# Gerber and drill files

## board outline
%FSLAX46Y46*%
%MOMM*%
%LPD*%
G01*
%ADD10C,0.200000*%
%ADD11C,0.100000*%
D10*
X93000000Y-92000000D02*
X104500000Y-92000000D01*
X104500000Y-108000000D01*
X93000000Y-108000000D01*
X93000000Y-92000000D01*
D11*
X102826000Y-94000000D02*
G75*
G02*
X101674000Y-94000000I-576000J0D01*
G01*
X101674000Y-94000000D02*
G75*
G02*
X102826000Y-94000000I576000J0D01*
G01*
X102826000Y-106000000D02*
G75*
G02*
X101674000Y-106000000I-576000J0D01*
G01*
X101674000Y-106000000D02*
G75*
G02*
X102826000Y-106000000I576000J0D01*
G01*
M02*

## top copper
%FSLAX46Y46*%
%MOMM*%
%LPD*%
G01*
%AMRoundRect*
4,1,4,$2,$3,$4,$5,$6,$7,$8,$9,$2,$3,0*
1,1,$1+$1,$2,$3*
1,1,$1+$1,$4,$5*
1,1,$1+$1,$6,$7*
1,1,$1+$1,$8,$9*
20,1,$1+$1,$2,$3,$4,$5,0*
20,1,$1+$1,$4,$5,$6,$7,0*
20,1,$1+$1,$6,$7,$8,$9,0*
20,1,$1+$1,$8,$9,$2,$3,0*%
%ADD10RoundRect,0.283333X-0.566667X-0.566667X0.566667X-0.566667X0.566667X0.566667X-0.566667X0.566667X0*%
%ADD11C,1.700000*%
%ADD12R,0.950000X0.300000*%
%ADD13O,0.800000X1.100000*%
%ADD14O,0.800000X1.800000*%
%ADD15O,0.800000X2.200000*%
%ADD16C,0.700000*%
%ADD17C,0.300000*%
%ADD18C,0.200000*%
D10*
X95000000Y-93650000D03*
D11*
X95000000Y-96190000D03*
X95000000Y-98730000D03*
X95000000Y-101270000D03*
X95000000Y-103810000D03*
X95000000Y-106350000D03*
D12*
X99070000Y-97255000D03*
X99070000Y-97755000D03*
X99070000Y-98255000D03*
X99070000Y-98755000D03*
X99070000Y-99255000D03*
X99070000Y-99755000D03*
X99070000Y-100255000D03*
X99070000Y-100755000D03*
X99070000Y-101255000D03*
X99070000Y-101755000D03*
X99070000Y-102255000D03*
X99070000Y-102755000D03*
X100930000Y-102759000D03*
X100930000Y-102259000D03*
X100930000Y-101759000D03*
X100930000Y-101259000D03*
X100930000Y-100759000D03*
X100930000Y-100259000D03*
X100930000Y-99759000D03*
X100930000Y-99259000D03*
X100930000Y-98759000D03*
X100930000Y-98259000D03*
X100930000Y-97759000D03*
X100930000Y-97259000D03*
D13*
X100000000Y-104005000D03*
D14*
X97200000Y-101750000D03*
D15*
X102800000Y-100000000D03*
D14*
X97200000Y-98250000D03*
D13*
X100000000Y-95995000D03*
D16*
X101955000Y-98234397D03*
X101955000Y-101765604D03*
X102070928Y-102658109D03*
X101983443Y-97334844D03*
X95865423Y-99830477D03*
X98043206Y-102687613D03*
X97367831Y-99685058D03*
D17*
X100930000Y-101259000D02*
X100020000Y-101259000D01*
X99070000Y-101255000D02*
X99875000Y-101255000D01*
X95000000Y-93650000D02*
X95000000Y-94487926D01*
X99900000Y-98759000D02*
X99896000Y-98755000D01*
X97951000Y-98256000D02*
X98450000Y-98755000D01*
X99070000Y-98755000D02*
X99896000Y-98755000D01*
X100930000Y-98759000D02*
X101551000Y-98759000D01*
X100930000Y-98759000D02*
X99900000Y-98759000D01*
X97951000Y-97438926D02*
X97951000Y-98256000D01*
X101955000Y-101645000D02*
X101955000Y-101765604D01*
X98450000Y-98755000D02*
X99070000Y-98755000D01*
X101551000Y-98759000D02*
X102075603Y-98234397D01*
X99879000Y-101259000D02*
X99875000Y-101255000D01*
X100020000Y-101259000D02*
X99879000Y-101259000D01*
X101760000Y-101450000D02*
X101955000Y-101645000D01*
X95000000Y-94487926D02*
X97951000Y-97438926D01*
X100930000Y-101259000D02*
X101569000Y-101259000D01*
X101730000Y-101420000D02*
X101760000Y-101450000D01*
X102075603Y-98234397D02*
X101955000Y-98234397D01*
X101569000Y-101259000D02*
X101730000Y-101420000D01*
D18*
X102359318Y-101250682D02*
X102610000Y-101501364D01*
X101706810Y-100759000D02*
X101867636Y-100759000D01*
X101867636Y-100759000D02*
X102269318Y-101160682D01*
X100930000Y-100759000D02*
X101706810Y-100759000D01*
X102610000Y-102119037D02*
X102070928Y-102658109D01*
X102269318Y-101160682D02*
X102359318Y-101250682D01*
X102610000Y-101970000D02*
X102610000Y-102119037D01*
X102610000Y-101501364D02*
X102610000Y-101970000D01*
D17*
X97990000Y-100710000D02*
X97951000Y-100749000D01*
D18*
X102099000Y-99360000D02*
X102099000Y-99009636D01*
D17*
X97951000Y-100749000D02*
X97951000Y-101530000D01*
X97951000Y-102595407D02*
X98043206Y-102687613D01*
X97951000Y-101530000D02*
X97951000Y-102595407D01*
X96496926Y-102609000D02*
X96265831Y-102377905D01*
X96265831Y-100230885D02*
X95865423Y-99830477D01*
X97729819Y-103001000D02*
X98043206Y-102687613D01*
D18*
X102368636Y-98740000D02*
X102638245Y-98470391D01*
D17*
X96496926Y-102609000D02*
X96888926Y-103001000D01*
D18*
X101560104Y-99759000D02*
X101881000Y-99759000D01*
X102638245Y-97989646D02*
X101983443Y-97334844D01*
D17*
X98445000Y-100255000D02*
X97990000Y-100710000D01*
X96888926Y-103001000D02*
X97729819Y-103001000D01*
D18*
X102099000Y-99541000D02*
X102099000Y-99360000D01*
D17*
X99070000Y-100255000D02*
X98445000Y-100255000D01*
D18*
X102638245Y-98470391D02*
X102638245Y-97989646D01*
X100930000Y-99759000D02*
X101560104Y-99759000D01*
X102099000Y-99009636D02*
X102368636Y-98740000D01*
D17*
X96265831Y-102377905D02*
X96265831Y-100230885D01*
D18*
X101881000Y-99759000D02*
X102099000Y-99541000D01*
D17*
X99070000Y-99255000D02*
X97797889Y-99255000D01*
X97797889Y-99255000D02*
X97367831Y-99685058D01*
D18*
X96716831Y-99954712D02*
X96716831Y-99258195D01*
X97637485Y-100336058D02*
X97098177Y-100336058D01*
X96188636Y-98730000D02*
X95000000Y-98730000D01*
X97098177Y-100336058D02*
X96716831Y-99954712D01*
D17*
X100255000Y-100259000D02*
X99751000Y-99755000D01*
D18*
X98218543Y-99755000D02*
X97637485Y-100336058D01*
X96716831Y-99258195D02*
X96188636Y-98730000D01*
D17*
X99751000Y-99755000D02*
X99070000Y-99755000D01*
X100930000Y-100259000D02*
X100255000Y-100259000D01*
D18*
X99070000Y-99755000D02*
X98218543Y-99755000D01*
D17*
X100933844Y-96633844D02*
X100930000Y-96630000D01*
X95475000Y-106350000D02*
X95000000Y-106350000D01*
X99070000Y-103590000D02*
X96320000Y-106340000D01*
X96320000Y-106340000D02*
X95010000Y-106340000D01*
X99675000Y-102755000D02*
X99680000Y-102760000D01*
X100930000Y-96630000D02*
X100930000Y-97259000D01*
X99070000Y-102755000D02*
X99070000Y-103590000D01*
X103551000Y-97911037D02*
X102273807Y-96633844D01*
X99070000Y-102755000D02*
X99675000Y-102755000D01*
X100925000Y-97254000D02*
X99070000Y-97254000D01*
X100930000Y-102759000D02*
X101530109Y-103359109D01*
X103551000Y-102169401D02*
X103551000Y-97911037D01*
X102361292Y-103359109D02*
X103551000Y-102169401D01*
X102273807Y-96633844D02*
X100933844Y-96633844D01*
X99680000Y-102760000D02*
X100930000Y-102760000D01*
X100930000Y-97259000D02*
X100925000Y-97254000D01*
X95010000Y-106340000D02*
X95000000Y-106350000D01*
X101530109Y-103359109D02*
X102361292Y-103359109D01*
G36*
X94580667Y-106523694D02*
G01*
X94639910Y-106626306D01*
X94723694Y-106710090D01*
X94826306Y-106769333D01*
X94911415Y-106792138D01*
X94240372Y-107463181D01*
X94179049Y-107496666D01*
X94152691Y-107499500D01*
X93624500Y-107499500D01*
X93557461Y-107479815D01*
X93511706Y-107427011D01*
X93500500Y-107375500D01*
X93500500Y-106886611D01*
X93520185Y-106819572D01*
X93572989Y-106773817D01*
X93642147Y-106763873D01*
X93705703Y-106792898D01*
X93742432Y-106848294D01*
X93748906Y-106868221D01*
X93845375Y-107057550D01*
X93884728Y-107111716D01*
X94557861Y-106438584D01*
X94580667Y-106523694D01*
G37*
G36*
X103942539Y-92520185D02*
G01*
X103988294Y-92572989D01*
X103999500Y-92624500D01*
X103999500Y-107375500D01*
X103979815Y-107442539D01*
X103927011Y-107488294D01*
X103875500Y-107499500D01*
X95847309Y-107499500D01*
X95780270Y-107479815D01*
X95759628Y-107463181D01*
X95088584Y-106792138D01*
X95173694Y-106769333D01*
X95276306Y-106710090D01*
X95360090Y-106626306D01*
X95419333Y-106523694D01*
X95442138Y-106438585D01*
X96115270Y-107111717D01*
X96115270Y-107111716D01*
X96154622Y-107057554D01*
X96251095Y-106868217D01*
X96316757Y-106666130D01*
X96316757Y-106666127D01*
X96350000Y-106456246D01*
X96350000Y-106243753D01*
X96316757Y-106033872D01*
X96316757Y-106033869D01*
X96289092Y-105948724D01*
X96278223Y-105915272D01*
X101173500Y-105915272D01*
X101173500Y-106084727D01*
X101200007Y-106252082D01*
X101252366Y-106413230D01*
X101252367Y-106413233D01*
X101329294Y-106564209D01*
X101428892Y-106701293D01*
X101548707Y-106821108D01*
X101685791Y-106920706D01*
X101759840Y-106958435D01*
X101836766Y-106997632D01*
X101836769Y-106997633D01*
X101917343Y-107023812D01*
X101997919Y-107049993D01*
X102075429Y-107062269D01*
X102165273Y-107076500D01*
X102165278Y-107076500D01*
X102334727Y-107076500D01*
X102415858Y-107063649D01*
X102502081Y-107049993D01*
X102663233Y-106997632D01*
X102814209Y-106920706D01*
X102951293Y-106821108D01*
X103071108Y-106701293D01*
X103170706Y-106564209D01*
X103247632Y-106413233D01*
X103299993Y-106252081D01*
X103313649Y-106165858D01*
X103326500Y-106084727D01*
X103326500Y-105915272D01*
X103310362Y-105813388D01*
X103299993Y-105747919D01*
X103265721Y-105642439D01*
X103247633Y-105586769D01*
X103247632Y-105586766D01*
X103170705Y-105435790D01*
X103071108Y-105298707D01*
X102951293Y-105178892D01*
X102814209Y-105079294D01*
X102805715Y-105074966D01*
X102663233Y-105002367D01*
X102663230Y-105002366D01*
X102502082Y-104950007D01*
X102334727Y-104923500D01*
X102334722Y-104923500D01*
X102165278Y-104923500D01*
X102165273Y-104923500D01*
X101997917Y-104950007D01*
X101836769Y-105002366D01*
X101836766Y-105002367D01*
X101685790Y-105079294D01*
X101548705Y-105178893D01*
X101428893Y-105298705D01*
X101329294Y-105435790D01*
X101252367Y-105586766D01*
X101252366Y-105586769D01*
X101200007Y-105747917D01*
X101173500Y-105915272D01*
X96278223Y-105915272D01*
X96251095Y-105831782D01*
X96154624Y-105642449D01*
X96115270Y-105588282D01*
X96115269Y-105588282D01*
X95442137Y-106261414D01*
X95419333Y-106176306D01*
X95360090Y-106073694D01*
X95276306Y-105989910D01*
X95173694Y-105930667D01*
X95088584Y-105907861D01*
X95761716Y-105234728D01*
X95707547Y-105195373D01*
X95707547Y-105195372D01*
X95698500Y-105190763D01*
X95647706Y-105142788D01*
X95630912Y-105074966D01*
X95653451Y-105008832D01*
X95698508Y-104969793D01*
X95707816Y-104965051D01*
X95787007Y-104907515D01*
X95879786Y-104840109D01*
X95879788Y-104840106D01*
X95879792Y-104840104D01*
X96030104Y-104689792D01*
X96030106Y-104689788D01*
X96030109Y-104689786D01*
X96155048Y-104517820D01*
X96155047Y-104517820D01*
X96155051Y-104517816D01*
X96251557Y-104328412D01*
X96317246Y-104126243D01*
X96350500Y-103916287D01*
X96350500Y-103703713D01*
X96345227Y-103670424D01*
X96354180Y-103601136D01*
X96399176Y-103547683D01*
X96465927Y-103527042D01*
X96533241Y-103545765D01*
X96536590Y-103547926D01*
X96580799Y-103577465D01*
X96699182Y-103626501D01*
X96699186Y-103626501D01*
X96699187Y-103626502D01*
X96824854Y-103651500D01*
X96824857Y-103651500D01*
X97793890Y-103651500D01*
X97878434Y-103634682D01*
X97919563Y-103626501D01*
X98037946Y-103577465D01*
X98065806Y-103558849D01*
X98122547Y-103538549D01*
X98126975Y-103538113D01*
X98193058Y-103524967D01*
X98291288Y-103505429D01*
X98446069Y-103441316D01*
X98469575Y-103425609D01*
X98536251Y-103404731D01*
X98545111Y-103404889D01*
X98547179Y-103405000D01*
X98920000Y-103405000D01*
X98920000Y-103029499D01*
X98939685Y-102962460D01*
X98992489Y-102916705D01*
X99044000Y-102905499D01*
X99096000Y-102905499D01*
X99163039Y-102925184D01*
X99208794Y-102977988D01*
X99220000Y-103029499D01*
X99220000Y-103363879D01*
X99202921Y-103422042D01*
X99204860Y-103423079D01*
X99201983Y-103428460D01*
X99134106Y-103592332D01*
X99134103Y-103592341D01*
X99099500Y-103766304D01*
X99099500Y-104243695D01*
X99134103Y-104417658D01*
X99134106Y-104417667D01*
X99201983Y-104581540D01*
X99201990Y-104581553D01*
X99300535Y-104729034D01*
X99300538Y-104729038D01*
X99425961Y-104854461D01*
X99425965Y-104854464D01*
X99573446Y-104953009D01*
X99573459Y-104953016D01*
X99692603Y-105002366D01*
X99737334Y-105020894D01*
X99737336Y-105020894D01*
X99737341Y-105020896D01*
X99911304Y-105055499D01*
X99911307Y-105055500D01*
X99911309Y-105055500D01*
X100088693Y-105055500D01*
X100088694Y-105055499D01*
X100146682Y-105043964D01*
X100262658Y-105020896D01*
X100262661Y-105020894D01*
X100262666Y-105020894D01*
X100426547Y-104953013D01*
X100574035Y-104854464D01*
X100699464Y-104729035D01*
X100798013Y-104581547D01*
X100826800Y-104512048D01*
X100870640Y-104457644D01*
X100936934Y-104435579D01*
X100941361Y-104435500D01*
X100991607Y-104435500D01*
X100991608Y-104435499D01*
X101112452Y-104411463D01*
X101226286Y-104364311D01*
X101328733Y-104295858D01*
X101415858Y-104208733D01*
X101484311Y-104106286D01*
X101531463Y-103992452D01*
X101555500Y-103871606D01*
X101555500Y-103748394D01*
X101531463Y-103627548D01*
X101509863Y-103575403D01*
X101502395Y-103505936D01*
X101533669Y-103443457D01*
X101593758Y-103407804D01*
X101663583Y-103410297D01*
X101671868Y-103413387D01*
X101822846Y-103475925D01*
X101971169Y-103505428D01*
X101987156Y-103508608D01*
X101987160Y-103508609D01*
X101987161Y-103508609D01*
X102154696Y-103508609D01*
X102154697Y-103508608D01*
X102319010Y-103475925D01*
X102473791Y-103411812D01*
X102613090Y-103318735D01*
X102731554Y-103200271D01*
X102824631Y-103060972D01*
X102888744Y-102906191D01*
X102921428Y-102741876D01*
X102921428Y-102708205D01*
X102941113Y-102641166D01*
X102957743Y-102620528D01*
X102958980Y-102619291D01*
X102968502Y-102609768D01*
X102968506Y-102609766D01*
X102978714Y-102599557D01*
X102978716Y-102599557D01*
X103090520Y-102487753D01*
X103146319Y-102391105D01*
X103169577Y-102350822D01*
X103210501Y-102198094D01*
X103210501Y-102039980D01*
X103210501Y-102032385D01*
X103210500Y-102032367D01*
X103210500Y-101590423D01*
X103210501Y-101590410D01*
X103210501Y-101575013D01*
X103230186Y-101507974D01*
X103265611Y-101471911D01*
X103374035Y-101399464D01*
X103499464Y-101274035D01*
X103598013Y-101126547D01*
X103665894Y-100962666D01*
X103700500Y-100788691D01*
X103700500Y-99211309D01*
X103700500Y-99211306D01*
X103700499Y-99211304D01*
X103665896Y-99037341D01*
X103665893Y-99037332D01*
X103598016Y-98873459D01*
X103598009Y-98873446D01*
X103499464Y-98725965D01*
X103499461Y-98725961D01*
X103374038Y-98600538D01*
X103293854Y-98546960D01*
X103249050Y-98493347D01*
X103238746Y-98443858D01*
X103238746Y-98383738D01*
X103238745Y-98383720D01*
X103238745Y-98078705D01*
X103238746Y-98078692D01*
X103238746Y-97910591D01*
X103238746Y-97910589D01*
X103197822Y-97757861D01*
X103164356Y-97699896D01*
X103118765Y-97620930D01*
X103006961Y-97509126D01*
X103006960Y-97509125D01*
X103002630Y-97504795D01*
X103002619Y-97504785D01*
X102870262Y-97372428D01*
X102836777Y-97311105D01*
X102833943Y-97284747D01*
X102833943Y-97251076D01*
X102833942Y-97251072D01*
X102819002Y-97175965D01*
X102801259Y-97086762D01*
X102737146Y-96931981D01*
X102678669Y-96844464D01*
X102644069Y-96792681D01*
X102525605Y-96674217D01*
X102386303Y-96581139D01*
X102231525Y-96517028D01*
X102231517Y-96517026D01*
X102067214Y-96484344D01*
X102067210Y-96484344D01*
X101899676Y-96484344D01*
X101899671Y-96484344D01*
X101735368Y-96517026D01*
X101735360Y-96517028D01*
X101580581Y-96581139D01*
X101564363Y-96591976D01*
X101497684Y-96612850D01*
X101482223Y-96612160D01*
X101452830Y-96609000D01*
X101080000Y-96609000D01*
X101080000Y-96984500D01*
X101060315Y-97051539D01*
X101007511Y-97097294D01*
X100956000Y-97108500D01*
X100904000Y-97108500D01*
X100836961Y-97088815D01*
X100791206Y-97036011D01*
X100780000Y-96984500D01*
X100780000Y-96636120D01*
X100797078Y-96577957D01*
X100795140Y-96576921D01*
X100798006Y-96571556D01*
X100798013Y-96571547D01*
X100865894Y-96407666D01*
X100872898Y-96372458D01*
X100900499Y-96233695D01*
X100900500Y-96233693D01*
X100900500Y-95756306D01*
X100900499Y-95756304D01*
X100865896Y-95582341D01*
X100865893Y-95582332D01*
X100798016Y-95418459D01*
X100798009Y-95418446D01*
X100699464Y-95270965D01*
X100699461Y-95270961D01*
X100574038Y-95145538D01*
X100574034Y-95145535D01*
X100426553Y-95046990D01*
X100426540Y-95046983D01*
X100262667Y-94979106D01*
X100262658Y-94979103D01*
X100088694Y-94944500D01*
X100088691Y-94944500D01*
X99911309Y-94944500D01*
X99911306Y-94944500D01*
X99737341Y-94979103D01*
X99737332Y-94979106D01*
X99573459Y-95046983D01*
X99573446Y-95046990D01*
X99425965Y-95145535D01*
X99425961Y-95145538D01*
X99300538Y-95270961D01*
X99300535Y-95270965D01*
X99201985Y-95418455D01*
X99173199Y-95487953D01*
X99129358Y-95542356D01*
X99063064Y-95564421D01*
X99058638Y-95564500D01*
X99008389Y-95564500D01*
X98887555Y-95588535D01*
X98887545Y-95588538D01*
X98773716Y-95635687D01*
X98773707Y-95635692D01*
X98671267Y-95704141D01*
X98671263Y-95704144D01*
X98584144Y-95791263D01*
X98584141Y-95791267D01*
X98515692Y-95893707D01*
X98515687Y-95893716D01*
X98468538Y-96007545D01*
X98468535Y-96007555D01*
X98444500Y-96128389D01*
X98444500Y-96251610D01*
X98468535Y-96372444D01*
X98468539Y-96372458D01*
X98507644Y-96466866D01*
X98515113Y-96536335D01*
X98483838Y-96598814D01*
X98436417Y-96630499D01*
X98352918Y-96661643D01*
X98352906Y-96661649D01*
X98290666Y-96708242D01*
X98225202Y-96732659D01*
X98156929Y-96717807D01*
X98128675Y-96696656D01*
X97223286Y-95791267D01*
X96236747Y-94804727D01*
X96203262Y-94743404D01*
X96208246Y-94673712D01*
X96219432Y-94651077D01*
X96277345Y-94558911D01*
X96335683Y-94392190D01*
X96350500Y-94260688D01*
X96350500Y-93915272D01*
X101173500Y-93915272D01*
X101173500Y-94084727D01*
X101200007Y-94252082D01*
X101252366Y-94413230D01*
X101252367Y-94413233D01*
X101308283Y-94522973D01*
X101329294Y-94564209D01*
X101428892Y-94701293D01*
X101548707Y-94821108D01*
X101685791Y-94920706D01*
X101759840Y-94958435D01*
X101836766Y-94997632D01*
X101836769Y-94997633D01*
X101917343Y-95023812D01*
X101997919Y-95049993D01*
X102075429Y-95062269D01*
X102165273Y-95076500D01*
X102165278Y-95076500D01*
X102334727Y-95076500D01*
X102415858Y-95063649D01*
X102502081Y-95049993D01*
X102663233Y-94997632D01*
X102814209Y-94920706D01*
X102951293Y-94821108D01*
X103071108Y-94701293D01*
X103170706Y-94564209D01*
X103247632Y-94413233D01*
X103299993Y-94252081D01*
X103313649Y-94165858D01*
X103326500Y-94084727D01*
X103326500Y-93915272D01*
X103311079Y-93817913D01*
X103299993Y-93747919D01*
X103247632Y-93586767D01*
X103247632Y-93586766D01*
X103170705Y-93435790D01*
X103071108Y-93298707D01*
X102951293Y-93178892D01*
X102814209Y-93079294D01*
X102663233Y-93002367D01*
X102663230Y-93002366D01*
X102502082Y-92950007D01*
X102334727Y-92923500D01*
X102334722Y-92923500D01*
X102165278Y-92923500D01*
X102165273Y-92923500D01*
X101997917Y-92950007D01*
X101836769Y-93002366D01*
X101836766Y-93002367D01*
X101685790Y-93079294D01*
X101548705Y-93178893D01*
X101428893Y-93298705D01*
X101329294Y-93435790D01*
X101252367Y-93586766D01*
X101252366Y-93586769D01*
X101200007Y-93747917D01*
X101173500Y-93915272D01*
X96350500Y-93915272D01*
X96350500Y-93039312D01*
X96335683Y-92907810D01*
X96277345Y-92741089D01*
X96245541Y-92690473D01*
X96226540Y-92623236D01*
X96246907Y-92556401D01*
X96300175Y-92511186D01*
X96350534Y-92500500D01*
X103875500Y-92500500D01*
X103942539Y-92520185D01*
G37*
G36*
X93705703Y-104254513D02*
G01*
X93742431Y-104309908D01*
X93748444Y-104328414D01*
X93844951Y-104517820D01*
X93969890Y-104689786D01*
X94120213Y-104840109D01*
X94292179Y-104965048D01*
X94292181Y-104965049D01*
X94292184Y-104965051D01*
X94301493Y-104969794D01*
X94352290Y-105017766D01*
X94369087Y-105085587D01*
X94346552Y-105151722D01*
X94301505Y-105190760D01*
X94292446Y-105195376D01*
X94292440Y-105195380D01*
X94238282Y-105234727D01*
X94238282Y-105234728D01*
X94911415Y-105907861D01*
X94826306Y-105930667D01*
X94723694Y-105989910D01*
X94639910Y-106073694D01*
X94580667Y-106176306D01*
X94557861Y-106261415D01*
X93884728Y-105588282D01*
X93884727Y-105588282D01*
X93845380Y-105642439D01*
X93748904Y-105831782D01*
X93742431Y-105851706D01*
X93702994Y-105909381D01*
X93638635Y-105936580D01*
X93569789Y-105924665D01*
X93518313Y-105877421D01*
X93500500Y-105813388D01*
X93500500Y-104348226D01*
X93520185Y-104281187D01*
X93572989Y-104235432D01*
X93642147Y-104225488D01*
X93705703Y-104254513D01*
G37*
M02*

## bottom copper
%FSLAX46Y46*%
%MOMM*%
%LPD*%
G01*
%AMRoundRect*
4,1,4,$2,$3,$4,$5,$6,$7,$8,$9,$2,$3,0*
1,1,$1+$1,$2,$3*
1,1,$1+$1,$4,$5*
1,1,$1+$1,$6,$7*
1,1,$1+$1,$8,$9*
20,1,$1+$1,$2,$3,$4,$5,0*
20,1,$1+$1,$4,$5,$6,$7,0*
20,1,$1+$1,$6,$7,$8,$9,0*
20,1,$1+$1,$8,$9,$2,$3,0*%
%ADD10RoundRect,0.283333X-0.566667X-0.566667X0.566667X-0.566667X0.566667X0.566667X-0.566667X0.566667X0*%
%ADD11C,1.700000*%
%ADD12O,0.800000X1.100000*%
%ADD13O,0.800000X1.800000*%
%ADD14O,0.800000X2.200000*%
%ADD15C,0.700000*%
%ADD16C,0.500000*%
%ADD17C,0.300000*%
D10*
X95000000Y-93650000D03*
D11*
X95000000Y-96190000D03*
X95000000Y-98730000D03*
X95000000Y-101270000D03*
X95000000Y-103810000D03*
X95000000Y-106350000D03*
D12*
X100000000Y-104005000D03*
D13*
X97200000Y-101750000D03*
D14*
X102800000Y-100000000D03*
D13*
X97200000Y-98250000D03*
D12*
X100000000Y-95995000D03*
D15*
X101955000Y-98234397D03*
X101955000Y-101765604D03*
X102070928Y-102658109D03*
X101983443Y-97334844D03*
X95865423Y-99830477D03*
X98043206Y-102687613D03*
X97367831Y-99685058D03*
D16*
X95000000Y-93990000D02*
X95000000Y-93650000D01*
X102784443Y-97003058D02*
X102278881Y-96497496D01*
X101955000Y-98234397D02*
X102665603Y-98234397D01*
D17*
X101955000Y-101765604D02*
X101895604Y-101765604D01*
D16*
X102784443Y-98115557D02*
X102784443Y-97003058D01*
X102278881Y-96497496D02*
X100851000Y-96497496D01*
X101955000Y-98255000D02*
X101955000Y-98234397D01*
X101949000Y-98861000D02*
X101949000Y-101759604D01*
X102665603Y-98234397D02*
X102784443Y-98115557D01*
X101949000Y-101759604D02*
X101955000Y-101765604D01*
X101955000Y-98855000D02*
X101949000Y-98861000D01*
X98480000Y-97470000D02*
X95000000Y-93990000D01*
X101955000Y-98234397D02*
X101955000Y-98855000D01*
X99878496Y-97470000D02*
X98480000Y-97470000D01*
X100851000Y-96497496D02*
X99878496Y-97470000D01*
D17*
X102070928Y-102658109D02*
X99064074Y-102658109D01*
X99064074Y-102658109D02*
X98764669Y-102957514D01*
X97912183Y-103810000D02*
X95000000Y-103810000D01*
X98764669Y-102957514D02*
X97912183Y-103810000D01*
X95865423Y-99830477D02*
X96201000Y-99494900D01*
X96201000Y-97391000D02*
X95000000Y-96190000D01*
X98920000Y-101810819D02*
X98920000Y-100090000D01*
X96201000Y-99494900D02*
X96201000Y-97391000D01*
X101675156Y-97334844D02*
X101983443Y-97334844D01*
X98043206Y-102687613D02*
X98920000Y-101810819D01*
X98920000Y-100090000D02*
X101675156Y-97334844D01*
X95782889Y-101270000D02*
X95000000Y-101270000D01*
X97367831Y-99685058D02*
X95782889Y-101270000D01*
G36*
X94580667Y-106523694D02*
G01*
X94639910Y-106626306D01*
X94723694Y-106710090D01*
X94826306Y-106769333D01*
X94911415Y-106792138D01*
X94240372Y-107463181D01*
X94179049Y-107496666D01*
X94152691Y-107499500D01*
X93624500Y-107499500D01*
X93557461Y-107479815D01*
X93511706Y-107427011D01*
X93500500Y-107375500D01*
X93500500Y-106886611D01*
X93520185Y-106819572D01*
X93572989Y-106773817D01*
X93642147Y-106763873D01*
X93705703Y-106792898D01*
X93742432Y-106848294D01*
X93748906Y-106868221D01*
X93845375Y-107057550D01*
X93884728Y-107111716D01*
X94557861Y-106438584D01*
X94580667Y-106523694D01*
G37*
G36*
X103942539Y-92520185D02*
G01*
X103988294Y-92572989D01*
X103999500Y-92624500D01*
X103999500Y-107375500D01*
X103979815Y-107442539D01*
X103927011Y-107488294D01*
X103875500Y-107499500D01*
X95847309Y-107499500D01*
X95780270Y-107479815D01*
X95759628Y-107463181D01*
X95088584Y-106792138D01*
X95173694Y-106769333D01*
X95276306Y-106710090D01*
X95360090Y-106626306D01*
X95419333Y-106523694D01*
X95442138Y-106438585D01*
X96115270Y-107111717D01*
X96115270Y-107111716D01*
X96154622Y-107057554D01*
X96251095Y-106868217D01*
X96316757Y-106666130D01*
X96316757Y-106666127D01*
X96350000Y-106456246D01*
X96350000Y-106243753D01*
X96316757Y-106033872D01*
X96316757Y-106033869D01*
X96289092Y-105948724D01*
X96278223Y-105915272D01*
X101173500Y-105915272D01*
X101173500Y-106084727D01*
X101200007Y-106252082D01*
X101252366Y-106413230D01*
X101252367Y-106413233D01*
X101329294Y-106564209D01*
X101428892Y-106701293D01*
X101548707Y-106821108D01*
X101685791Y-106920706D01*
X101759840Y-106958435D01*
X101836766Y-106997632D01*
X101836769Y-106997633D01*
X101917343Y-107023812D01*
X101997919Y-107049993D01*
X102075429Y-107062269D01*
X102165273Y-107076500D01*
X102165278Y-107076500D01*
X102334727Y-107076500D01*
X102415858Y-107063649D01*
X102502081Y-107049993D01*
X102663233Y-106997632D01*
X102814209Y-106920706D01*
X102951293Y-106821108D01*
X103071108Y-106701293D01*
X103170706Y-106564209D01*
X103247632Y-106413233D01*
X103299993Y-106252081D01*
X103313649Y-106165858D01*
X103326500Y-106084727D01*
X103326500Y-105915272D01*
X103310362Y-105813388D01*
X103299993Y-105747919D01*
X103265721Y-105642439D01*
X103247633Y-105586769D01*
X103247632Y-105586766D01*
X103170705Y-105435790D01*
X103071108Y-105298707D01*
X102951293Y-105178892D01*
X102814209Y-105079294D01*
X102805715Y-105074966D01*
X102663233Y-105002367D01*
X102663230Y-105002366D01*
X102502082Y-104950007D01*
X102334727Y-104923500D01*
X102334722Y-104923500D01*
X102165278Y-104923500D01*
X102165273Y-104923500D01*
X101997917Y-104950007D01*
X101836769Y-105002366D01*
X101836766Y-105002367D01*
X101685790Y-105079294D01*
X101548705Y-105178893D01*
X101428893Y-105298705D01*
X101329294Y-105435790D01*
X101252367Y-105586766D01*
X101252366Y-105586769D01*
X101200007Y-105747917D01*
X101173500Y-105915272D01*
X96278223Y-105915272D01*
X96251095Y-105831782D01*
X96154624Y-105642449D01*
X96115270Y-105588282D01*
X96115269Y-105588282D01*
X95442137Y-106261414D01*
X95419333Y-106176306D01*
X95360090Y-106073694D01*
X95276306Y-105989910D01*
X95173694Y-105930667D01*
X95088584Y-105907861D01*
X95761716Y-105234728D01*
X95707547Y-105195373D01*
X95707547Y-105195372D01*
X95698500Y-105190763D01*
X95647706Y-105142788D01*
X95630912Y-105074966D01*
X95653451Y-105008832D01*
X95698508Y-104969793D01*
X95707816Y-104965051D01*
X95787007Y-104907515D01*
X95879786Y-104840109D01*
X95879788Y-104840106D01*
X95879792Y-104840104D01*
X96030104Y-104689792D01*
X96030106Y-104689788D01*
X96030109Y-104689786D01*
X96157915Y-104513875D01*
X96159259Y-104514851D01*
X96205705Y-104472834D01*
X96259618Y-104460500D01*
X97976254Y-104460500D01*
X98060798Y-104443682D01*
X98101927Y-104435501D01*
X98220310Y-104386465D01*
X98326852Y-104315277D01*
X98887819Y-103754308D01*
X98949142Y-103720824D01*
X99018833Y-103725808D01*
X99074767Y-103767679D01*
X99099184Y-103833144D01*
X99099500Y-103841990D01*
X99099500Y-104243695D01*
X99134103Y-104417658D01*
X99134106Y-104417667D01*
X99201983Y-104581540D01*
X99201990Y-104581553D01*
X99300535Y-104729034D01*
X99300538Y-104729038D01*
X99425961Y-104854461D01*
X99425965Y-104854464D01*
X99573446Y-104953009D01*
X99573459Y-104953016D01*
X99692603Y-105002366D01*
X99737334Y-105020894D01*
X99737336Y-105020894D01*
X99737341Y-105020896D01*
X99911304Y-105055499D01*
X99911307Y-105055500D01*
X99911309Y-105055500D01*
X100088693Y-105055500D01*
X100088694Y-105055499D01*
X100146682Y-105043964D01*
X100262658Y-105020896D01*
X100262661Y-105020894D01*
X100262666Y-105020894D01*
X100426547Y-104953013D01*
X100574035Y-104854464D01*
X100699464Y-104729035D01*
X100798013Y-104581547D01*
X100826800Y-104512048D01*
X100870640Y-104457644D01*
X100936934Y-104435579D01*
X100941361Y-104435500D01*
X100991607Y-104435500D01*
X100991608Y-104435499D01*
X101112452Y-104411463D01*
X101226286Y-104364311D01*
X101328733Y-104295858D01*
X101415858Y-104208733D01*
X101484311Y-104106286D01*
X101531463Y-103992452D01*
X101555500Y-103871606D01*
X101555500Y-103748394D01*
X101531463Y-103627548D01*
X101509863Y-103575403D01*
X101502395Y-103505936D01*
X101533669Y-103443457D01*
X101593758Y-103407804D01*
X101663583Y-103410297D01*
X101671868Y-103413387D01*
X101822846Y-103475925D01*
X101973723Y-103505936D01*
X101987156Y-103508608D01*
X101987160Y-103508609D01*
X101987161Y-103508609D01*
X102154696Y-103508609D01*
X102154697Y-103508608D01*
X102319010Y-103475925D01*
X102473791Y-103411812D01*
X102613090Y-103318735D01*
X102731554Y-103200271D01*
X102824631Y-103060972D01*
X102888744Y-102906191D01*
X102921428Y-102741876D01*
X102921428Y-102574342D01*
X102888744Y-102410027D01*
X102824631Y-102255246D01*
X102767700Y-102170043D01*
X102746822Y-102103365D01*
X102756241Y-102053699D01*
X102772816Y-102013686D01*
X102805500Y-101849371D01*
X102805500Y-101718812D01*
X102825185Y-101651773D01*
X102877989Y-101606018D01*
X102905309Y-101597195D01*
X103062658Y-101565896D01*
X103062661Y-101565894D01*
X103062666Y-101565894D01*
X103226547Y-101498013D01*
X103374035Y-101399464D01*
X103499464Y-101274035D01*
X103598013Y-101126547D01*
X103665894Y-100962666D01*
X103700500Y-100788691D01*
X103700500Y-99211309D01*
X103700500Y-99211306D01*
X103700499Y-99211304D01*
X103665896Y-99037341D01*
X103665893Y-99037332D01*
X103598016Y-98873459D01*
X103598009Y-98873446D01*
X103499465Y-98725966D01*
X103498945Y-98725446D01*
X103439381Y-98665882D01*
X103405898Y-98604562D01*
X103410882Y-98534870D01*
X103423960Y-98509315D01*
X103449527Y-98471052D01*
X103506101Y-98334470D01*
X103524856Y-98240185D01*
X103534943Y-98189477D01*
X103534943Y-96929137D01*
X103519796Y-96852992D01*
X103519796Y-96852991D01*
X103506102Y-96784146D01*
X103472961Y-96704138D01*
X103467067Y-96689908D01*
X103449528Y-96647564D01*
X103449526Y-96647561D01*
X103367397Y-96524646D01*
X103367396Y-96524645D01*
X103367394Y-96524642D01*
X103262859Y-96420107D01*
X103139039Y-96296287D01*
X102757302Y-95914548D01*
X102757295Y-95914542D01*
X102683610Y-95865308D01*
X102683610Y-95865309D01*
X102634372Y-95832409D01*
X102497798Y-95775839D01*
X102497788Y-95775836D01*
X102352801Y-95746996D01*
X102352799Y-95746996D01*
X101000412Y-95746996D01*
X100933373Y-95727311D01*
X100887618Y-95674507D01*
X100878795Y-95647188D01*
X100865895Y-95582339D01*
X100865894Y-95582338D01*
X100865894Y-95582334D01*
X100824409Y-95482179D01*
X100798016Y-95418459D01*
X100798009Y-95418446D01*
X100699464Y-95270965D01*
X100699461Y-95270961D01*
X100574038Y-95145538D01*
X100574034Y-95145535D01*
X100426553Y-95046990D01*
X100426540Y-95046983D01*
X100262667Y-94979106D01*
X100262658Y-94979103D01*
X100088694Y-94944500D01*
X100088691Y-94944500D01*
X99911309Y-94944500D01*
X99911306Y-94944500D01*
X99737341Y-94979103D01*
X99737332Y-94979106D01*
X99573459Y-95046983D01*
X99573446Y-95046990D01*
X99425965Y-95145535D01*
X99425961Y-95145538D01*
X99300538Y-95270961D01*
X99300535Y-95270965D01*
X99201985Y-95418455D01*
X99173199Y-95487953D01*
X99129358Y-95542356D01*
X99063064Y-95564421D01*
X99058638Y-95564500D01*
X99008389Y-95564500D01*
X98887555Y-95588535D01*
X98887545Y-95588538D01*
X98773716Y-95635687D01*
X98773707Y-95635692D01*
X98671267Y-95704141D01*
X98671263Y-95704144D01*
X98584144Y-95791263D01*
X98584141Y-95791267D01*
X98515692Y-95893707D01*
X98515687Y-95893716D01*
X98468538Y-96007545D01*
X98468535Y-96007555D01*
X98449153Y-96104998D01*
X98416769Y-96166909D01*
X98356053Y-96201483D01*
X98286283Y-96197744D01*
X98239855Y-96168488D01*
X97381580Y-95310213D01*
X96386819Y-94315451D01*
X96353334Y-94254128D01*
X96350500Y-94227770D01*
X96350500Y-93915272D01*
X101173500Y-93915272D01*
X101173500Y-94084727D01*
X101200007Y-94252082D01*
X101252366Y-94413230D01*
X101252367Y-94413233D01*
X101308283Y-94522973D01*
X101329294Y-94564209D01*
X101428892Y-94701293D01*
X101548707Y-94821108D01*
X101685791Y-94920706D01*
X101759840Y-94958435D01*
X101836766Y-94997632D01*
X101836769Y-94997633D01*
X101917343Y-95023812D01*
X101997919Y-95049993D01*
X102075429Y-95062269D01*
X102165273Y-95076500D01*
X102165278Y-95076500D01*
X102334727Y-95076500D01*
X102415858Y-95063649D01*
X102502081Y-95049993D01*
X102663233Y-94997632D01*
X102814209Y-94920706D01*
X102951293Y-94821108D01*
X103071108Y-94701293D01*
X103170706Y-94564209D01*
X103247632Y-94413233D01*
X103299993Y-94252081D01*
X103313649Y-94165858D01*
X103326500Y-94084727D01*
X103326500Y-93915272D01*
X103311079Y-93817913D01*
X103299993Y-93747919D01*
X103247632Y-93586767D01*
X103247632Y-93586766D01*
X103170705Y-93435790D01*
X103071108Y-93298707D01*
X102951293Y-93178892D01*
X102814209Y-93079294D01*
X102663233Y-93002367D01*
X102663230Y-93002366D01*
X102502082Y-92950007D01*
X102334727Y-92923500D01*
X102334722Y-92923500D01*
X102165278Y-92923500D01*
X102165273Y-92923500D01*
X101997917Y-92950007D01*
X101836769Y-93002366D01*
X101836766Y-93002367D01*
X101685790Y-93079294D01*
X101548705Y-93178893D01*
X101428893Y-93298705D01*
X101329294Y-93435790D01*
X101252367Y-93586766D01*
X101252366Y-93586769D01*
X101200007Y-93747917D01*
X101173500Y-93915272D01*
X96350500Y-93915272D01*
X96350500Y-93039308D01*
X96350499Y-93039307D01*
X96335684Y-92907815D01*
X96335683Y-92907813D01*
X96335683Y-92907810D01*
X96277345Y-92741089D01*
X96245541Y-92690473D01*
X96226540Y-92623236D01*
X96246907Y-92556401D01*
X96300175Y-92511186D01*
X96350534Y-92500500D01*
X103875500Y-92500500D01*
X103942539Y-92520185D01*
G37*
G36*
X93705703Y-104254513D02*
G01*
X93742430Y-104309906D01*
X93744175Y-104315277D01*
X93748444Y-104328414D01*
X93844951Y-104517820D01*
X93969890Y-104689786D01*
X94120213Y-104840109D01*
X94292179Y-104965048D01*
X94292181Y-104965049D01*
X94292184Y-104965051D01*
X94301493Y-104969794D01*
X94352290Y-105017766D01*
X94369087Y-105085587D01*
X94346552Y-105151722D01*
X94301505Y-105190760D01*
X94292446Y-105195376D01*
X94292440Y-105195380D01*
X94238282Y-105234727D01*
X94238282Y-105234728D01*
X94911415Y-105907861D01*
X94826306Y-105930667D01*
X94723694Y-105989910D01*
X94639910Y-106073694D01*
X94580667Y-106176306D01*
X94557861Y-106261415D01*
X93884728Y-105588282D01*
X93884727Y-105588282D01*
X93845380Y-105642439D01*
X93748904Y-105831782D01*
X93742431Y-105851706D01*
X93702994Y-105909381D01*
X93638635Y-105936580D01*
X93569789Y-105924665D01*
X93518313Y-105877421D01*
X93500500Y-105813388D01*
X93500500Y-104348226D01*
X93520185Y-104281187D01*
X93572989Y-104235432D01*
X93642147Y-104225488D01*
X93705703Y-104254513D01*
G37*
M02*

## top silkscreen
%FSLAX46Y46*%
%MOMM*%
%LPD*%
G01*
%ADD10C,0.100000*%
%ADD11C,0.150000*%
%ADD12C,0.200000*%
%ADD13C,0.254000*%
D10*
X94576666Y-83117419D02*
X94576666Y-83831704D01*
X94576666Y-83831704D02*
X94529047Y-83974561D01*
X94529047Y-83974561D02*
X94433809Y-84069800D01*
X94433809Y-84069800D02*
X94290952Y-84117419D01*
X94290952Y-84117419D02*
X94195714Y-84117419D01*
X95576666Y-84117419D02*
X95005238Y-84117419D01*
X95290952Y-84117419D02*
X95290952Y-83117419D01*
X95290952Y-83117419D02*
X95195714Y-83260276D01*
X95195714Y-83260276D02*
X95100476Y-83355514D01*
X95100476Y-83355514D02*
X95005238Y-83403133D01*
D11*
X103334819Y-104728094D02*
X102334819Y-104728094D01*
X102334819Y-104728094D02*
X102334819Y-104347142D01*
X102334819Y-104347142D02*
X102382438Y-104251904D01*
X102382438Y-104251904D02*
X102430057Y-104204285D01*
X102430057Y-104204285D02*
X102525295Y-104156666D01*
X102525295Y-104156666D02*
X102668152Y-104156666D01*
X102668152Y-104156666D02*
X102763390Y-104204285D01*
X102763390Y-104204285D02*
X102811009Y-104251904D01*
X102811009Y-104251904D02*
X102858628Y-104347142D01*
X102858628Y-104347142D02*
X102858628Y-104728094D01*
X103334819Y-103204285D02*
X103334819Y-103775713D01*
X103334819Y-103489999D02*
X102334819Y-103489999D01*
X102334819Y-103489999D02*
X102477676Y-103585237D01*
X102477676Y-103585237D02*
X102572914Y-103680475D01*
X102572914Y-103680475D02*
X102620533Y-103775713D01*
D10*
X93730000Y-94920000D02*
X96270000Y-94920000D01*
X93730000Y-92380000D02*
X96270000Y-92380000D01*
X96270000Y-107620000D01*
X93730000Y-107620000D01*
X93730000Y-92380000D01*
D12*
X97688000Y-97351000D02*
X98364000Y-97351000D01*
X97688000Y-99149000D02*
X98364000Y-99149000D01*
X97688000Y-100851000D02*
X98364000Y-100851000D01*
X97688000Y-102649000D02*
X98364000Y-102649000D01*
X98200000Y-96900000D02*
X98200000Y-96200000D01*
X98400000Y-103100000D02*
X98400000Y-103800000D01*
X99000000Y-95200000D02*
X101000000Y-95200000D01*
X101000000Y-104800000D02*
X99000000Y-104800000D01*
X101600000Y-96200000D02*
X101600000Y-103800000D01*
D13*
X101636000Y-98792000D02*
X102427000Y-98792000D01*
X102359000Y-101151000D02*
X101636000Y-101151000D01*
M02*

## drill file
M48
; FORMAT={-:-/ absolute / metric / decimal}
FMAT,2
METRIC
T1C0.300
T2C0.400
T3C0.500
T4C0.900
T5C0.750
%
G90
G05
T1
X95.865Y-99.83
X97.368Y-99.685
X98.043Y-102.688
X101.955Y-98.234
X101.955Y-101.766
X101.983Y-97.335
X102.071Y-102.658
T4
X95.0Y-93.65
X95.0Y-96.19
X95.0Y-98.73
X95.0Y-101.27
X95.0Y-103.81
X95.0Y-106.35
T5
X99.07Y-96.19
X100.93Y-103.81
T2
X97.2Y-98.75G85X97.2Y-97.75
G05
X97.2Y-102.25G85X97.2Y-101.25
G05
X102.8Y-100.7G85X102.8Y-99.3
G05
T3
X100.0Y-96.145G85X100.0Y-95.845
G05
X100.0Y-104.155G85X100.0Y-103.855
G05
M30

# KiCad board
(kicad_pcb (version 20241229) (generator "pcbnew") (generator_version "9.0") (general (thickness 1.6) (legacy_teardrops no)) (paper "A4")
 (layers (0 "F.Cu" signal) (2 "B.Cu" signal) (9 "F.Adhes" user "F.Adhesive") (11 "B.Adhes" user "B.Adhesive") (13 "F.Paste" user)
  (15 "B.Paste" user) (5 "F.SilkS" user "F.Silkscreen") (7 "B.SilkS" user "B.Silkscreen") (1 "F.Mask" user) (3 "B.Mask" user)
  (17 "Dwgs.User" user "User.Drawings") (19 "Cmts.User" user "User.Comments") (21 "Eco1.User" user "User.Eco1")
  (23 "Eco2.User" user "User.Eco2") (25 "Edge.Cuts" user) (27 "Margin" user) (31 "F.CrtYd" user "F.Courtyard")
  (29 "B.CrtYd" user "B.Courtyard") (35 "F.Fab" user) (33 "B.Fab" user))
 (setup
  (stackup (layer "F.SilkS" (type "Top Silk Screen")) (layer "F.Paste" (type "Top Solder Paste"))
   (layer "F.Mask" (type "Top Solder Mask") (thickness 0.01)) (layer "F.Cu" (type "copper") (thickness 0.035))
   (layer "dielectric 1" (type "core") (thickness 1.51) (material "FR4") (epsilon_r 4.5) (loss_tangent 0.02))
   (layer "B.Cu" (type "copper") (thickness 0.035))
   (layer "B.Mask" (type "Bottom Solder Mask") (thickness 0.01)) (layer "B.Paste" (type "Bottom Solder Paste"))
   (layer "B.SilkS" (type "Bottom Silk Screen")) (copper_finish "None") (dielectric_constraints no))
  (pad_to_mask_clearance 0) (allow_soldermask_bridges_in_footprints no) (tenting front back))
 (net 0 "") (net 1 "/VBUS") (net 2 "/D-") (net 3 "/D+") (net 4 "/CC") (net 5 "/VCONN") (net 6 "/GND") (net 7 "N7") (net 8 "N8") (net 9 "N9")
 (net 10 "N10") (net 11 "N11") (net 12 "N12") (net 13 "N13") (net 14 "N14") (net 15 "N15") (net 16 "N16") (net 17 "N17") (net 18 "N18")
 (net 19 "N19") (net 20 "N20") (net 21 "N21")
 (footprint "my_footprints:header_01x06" (layer "F.Cu") (at 95 100)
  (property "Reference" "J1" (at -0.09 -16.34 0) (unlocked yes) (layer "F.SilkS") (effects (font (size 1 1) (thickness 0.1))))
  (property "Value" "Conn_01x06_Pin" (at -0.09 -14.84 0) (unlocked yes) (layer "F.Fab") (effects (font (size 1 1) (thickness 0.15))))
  (fp_line (start -1.27 -5.08) (end 1.27 -5.08) (stroke (width 0.1) (type default)) (layer "F.SilkS"))
  (fp_rect (start -1.27 -7.62) (end 1.27 7.62) (stroke (width 0.1) (type default)) (fill no) (layer "F.SilkS"))
  (pad "1" thru_hole roundrect (at 0 -6.35) (size 1.7 1.7) (drill 0.9) (layers "*.Cu" "F.Mask" "F.Paste") (remove_unused_layers no)
   (roundrect_rratio 0.1666666667) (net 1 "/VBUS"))
  (pad "2" thru_hole circle (at 0 -3.81) (size 1.7 1.7) (drill 0.9) (layers "*.Cu" "F.Mask" "F.Paste") (remove_unused_layers no)
   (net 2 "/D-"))
  (pad "3" thru_hole circle (at 0 -1.27) (size 1.7 1.7) (drill 0.9) (layers "*.Cu" "F.Mask" "F.Paste") (remove_unused_layers no)
   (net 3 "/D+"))
  (pad "4" thru_hole circle (at 0 1.27) (size 1.7 1.7) (drill 0.9) (layers "*.Cu" "F.Mask" "F.Paste") (remove_unused_layers no)
   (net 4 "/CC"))
  (pad "5" thru_hole circle (at 0 3.81) (size 1.7 1.7) (drill 0.9) (layers "*.Cu" "F.Mask" "F.Paste") (remove_unused_layers no)
   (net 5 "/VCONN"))
  (pad "6" thru_hole circle (at 0 6.35) (size 1.7 1.7) (drill 0.9) (layers "*.Cu" "F.Mask" "F.Paste") (remove_unused_layers no)
   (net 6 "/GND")))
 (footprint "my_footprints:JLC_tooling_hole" (layer "F.Cu") (at 102.25 94)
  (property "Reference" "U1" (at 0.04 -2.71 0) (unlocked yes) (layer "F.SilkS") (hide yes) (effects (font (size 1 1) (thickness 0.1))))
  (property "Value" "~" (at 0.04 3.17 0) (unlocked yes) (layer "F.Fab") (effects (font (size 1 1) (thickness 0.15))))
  (fp_circle (center 0 0) (end 0.576 0) (stroke (width 0.1) (type default)) (fill no) (layer "Edge.Cuts")))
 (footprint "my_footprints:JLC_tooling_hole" (layer "F.Cu") (at 102.25 106)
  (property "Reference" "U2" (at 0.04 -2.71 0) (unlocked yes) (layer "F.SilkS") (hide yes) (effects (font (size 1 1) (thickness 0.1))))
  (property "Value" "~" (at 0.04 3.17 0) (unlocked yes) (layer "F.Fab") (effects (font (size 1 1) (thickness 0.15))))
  (fp_circle (center 0 0) (end 0.576 0) (stroke (width 0.1) (type default)) (fill no) (layer "Edge.Cuts")))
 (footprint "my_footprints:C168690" (layer "F.Cu") (at 100 100 90)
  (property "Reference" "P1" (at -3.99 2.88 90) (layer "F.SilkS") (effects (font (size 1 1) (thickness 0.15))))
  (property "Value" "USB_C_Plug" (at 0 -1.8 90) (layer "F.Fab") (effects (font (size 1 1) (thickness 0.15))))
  (fp_line (start 2.649 -2.312) (end 2.649 -1.636) (stroke (width 0.2) (type solid)) (layer "F.SilkS"))
  (fp_line (start 0.851 -2.312) (end 0.851 -1.636) (stroke (width 0.2) (type solid)) (layer "F.SilkS"))
  (fp_line (start -0.851 -2.312) (end -0.851 -1.636) (stroke (width 0.2) (type solid)) (layer "F.SilkS"))
  (fp_line (start -2.649 -2.312) (end -2.649 -1.636) (stroke (width 0.2) (type solid)) (layer "F.SilkS"))
  (fp_line (start 3.1 -1.8) (end 3.8 -1.8) (stroke (width 0.2) (type solid)) (layer "F.SilkS"))
  (fp_line (start -3.1 -1.6) (end -3.8 -1.6) (stroke (width 0.2) (type solid)) (layer "F.SilkS"))
  (fp_line (start 4.8 -1) (end 4.8 1) (stroke (width 0.2) (type solid)) (layer "F.SilkS"))
  (fp_line (start -4.8 1) (end -4.8 -1) (stroke (width 0.2) (type solid)) (layer "F.SilkS"))
  (fp_line (start 3.8 1.6) (end -3.8 1.6) (stroke (width 0.2) (type solid)) (layer "F.SilkS"))
  (fp_line (start 1.208 1.636) (end 1.208 2.427) (stroke (width 0.254) (type solid)) (layer "F.SilkS"))
  (fp_line (start -1.151 2.359) (end -1.151 1.636) (stroke (width 0.254) (type solid)) (layer "F.SilkS"))
  (pad "" np_thru_hole circle (at -3.81 0.93 90) (size 0.75 0.75) (drill 0.75) (layers "*.Mask"))
  (pad "" np_thru_hole circle (at 3.81 -0.93 90) (size 0.75 0.75) (drill 0.75) (layers "*.Mask"))
  (pad "A1" smd rect (at 2.745 -0.93 90) (size 0.3 0.95) (layers "F.Cu" "F.Mask" "F.Paste") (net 6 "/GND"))
  (pad "A2" smd rect (at 2.245 -0.93 90) (size 0.3 0.95) (layers "F.Cu" "F.Mask" "F.Paste") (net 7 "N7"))
  (pad "A3" smd rect (at 1.745 -0.93 90) (size 0.3 0.95) (layers "F.Cu" "F.Mask" "F.Paste") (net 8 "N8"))
  (pad "A4" smd rect (at 1.245 -0.93 90) (size 0.3 0.95) (layers "F.Cu" "F.Mask" "F.Paste") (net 1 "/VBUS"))
  (pad "A5" smd rect (at 0.745 -0.93 90) (size 0.3 0.95) (layers "F.Cu" "F.Mask" "F.Paste") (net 4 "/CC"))
  (pad "A6" smd rect (at 0.245 -0.93 90) (size 0.3 0.95) (layers "F.Cu" "F.Mask" "F.Paste") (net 3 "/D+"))
  (pad "A7" smd rect (at -0.255 -0.93 90) (size 0.3 0.95) (layers "F.Cu" "F.Mask" "F.Paste") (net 2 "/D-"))
  (pad "A8" smd rect (at -0.755 -0.93 90) (size 0.3 0.95) (layers "F.Cu" "F.Mask" "F.Paste") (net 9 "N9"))
  (pad "A9" smd rect (at -1.255 -0.93 90) (size 0.3 0.95) (layers "F.Cu" "F.Mask" "F.Paste") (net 1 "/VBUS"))
  (pad "A10" smd rect (at -1.755 -0.93 90) (size 0.3 0.95) (layers "F.Cu" "F.Mask" "F.Paste") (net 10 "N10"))
  (pad "A11" smd rect (at -2.255 -0.93 90) (size 0.3 0.95) (layers "F.Cu" "F.Mask" "F.Paste") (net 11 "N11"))
  (pad "A12" smd rect (at -2.755 -0.93 90) (size 0.3 0.95) (layers "F.Cu" "F.Mask" "F.Paste") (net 6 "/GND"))
  (pad "B1" smd rect (at -2.759 0.93 90) (size 0.3 0.95) (layers "F.Cu" "F.Mask" "F.Paste") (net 6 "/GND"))
  (pad "B2" smd rect (at -2.259 0.93 90) (size 0.3 0.95) (layers "F.Cu" "F.Mask" "F.Paste") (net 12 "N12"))
  (pad "B3" smd rect (at -1.759 0.93 90) (size 0.3 0.95) (layers "F.Cu" "F.Mask" "F.Paste") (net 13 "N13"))
  (pad "B4" smd rect (at -1.259 0.93 90) (size 0.3 0.95) (layers "F.Cu" "F.Mask" "F.Paste") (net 1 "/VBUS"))
  (pad "B5" smd rect (at -0.759 0.93 90) (size 0.3 0.95) (layers "F.Cu" "F.Mask" "F.Paste") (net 5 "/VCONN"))
  (pad "B6" smd rect (at -0.259 0.93 90) (size 0.3 0.95) (layers "F.Cu" "F.Mask" "F.Paste") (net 3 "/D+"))
  (pad "B7" smd rect (at 0.241 0.93 90) (size 0.3 0.95) (layers "F.Cu" "F.Mask" "F.Paste") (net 2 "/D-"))
  (pad "B8" smd rect (at 0.741 0.93 90) (size 0.3 0.95) (layers "F.Cu" "F.Mask" "F.Paste") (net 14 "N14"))
  (pad "B9" smd rect (at 1.241 0.93 90) (size 0.3 0.95) (layers "F.Cu" "F.Mask" "F.Paste") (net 1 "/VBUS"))
  (pad "B10" smd rect (at 1.741 0.93 90) (size 0.3 0.95) (layers "F.Cu" "F.Mask" "F.Paste") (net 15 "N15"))
  (pad "B11" smd rect (at 2.241 0.93 90) (size 0.3 0.95) (layers "F.Cu" "F.Mask" "F.Paste") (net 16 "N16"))
  (pad "B12" smd rect (at 2.741 0.93 90) (size 0.3 0.95) (layers "F.Cu" "F.Mask" "F.Paste") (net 6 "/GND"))
  (pad "S1" thru_hole oval (at -4.005 0 180) (size 0.8 1.1) (drill oval 0.5 0.8) (layers "*.Cu" "*.Mask") (remove_unused_layers no)
   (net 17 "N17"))
  (pad "S1" thru_hole oval (at -1.75 -2.8 180) (size 0.8 1.8) (drill oval 0.4 1.4) (layers "*.Cu" "*.Mask") (remove_unused_layers no)
   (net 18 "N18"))
  (pad "S1" thru_hole oval (at 0 2.8 180) (size 0.8 2.2) (drill oval 0.4 1.8) (layers "*.Cu" "*.Mask") (remove_unused_layers no)
   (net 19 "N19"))
  (pad "S1" thru_hole oval (at 1.75 -2.8 180) (size 0.8 1.8) (drill oval 0.4 1.4) (layers "*.Cu" "*.Mask") (remove_unused_layers no)
   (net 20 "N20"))
  (pad "S1" thru_hole oval (at 4.005 0 180) (size 0.8 1.1) (drill oval 0.5 0.8) (layers "*.Cu" "*.Mask") (remove_unused_layers no)
   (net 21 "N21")))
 (gr_rect (start 93 92) (end 104.5 108) (stroke (width 0.2) (type solid)) (fill no) (layer "Edge.Cuts"))
 (segment (start 100.93 101.259) (end 100.02 101.259) (width 0.3) (layer "F.Cu") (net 1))
 (segment (start 99.07 101.255) (end 99.875 101.255) (width 0.3) (layer "F.Cu") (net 1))
 (segment (start 95 93.65) (end 95 94.487926) (width 0.3) (layer "F.Cu") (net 1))
 (segment (start 99.9 98.759) (end 99.896 98.755) (width 0.3) (layer "F.Cu") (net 1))
 (segment (start 97.951 98.256) (end 98.45 98.755) (width 0.3) (layer "F.Cu") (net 1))
 (segment (start 99.07 98.755) (end 99.896 98.755) (width 0.3) (layer "F.Cu") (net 1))
 (segment (start 100.93 98.759) (end 101.551 98.759) (width 0.3) (layer "F.Cu") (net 1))
 (segment (start 100.93 98.759) (end 99.9 98.759) (width 0.3) (layer "F.Cu") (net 1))
 (segment (start 97.951 97.438926) (end 97.951 98.256) (width 0.3) (layer "F.Cu") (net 1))
 (segment (start 101.955 101.645) (end 101.955 101.765604) (width 0.3) (layer "F.Cu") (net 1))
 (segment (start 98.45 98.755) (end 99.07 98.755) (width 0.3) (layer "F.Cu") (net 1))
 (segment (start 101.551 98.759) (end 102.075603 98.234397) (width 0.3) (layer "F.Cu") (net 1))
 (segment (start 99.879 101.259) (end 99.875 101.255) (width 0.3) (layer "F.Cu") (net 1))
 (segment (start 100.02 101.259) (end 99.879 101.259) (width 0.3) (layer "F.Cu") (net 1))
 (segment (start 101.76 101.45) (end 101.955 101.645) (width 0.3) (layer "F.Cu") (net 1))
 (segment (start 95 94.487926) (end 97.951 97.438926) (width 0.3) (layer "F.Cu") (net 1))
 (segment (start 100.93 101.259) (end 101.569 101.259) (width 0.3) (layer "F.Cu") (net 1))
 (segment (start 101.73 101.42) (end 101.76 101.45) (width 0.3) (layer "F.Cu") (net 1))
 (segment (start 102.075603 98.234397) (end 101.955 98.234397) (width 0.3) (layer "F.Cu") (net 1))
 (segment (start 101.569 101.259) (end 101.73 101.42) (width 0.3) (layer "F.Cu") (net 1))
 (via (at 101.955 98.234397) (size 0.7) (drill 0.3) (layers "F.Cu" "B.Cu") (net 1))
 (via (at 101.955 101.765604) (size 0.7) (drill 0.3) (layers "F.Cu" "B.Cu") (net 1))
 (segment (start 95 93.99) (end 95 93.65) (width 0.5) (layer "B.Cu") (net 1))
 (segment (start 102.784443 97.003058) (end 102.278881 96.497496) (width 0.5) (layer "B.Cu") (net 1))
 (segment (start 101.955 98.234397) (end 102.665603 98.234397) (width 0.5) (layer "B.Cu") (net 1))
 (segment (start 101.955 101.765604) (end 101.895604 101.765604) (width 0.3) (layer "B.Cu") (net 1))
 (segment (start 102.784443 98.115557) (end 102.784443 97.003058) (width 0.5) (layer "B.Cu") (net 1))
 (segment (start 102.278881 96.497496) (end 100.851 96.497496) (width 0.5) (layer "B.Cu") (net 1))
 (segment (start 101.955 98.255) (end 101.955 98.234397) (width 0.5) (layer "B.Cu") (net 1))
 (segment (start 101.949 98.861) (end 101.949 101.759604) (width 0.5) (layer "B.Cu") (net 1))
 (segment (start 102.665603 98.234397) (end 102.784443 98.115557) (width 0.5) (layer "B.Cu") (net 1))
 (segment (start 101.949 101.759604) (end 101.955 101.765604) (width 0.5) (layer "B.Cu") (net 1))
 (segment (start 101.955 98.855) (end 101.949 98.861) (width 0.5) (layer "B.Cu") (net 1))
 (segment (start 98.48 97.47) (end 95 93.99) (width 0.5) (layer "B.Cu") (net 1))
 (segment (start 101.955 98.234397) (end 101.955 98.855) (width 0.5) (layer "B.Cu") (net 1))
 (segment (start 99.878496 97.47) (end 98.48 97.47) (width 0.5) (layer "B.Cu") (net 1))
 (segment (start 100.851 96.497496) (end 99.878496 97.47) (width 0.5) (layer "B.Cu") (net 1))
 (segment (start 102.359318 101.250682) (end 102.61 101.501364) (width 0.2) (layer "F.Cu") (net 5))
 (segment (start 101.70681 100.759) (end 101.867636 100.759) (width 0.2) (layer "F.Cu") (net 5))
 (segment (start 101.867636 100.759) (end 102.269318 101.160682) (width 0.2) (layer "F.Cu") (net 5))
 (segment (start 100.93 100.759) (end 101.70681 100.759) (width 0.2) (layer "F.Cu") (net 5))
 (segment (start 102.61 102.119037) (end 102.070928 102.658109) (width 0.2) (layer "F.Cu") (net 5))
 (segment (start 102.269318 101.160682) (end 102.359318 101.250682) (width 0.2) (layer "F.Cu") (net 5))
 (segment (start 102.61 101.97) (end 102.61 102.119037) (width 0.2) (layer "F.Cu") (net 5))
 (segment (start 102.61 101.501364) (end 102.61 101.97) (width 0.2) (layer "F.Cu") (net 5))
 (via (at 102.070928 102.658109) (size 0.7) (drill 0.3) (layers "F.Cu" "B.Cu") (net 5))
 (segment (start 102.070928 102.658109) (end 99.064074 102.658109) (width 0.3) (layer "B.Cu") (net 5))
 (segment (start 99.064074 102.658109) (end 98.764669 102.957514) (width 0.3) (layer "B.Cu") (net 5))
 (segment (start 97.912183 103.81) (end 95 103.81) (width 0.3) (layer "B.Cu") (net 5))
 (segment (start 98.764669 102.957514) (end 97.912183 103.81) (width 0.3) (layer "B.Cu") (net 5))
 (segment (start 97.99 100.71) (end 97.951 100.749) (width 0.3) (layer "F.Cu") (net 2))
 (segment (start 102.099 99.36) (end 102.099 99.009636) (width 0.2) (layer "F.Cu") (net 2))
 (segment (start 97.951 100.749) (end 97.951 101.53) (width 0.3) (layer "F.Cu") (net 2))
 (segment (start 97.951 102.595407) (end 98.043206 102.687613) (width 0.3) (layer "F.Cu") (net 2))
 (segment (start 97.951 101.53) (end 97.951 102.595407) (width 0.3) (layer "F.Cu") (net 2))
 (segment (start 96.496926 102.609) (end 96.265831 102.377905) (width 0.3) (layer "F.Cu") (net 2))
 (segment (start 96.265831 100.230885) (end 95.865423 99.830477) (width 0.3) (layer "F.Cu") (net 2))
 (segment (start 97.729819 103.001) (end 98.043206 102.687613) (width 0.3) (layer "F.Cu") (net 2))
 (segment (start 102.368636 98.74) (end 102.638245 98.470391) (width 0.2) (layer "F.Cu") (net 2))
 (segment (start 96.496926 102.609) (end 96.888926 103.001) (width 0.3) (layer "F.Cu") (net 2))
 (segment (start 101.560104 99.759) (end 101.881 99.759) (width 0.2) (layer "F.Cu") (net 2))
 (segment (start 102.638245 97.989646) (end 101.983443 97.334844) (width 0.2) (layer "F.Cu") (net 2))
 (segment (start 98.445 100.255) (end 97.99 100.71) (width 0.3) (layer "F.Cu") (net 2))
 (segment (start 96.888926 103.001) (end 97.729819 103.001) (width 0.3) (layer "F.Cu") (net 2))
 (segment (start 102.099 99.541) (end 102.099 99.36) (width 0.2) (layer "F.Cu") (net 2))
 (segment (start 99.07 100.255) (end 98.445 100.255) (width 0.3) (layer "F.Cu") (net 2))
 (segment (start 102.638245 98.470391) (end 102.638245 97.989646) (width 0.2) (layer "F.Cu") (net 2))
 (segment (start 100.93 99.759) (end 101.560104 99.759) (width 0.2) (layer "F.Cu") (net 2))
 (segment (start 102.099 99.009636) (end 102.368636 98.74) (width 0.2) (layer "F.Cu") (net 2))
 (segment (start 96.265831 102.377905) (end 96.265831 100.230885) (width 0.3) (layer "F.Cu") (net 2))
 (segment (start 101.881 99.759) (end 102.099 99.541) (width 0.2) (layer "F.Cu") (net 2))
 (via (at 101.983443 97.334844) (size 0.7) (drill 0.3) (layers "F.Cu" "B.Cu") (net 2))
 (via (at 95.865423 99.830477) (size 0.7) (drill 0.3) (layers "F.Cu" "B.Cu") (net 2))
 (via (at 98.043206 102.687613) (size 0.7) (drill 0.3) (layers "F.Cu" "B.Cu") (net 2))
 (segment (start 95.865423 99.830477) (end 96.201 99.4949) (width 0.3) (layer "B.Cu") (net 2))
 (segment (start 96.201 97.391) (end 95 96.19) (width 0.3) (layer "B.Cu") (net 2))
 (segment (start 98.92 101.810819) (end 98.92 100.09) (width 0.3) (layer "B.Cu") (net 2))
 (segment (start 96.201 99.4949) (end 96.201 97.391) (width 0.3) (layer "B.Cu") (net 2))
 (segment (start 101.675156 97.334844) (end 101.983443 97.334844) (width 0.3) (layer "B.Cu") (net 2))
 (segment (start 98.043206 102.687613) (end 98.92 101.810819) (width 0.3) (layer "B.Cu") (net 2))
 (segment (start 98.92 100.09) (end 101.675156 97.334844) (width 0.3) (layer "B.Cu") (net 2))
 (segment (start 99.07 99.255) (end 97.797889 99.255) (width 0.3) (layer "F.Cu") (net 4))
 (segment (start 97.797889 99.255) (end 97.367831 99.685058) (width 0.3) (layer "F.Cu") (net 4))
 (via (at 97.367831 99.685058) (size 0.7) (drill 0.3) (layers "F.Cu" "B.Cu") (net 4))
 (segment (start 95.782889 101.27) (end 95 101.27) (width 0.3) (layer "B.Cu") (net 4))
 (segment (start 97.367831 99.685058) (end 95.782889 101.27) (width 0.3) (layer "B.Cu") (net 4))
 (segment (start 96.716831 99.954712) (end 96.716831 99.258195) (width 0.2) (layer "F.Cu") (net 3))
 (segment (start 97.637485 100.336058) (end 97.098177 100.336058) (width 0.2) (layer "F.Cu") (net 3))
 (segment (start 96.188636 98.73) (end 95 98.73) (width 0.2) (layer "F.Cu") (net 3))
 (segment (start 97.098177 100.336058) (end 96.716831 99.954712) (width 0.2) (layer "F.Cu") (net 3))
 (segment (start 100.255 100.259) (end 99.751 99.755) (width 0.3) (layer "F.Cu") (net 3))
 (segment (start 98.218543 99.755) (end 97.637485 100.336058) (width 0.2) (layer "F.Cu") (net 3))
 (segment (start 96.716831 99.258195) (end 96.188636 98.73) (width 0.2) (layer "F.Cu") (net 3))
 (segment (start 99.751 99.755) (end 99.07 99.755) (width 0.3) (layer "F.Cu") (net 3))
 (segment (start 100.93 100.259) (end 100.255 100.259) (width 0.3) (layer "F.Cu") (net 3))
 (segment (start 99.07 99.755) (end 98.218543 99.755) (width 0.2) (layer "F.Cu") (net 3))
 (segment (start 100.933844 96.633844) (end 100.93 96.63) (width 0.3) (layer "F.Cu") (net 6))
 (segment (start 95.475 106.35) (end 95 106.35) (width 0.3) (layer "F.Cu") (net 6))
 (segment (start 99.07 103.59) (end 96.32 106.34) (width 0.3) (layer "F.Cu") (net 6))
 (segment (start 96.32 106.34) (end 95.01 106.34) (width 0.3) (layer "F.Cu") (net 6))
 (segment (start 99.675 102.755) (end 99.68 102.76) (width 0.3) (layer "F.Cu") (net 6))
 (segment (start 100.93 96.63) (end 100.93 97.259) (width 0.3) (layer "F.Cu") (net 6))
 (segment (start 99.07 102.755) (end 99.07 103.59) (width 0.3) (layer "F.Cu") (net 6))
 (segment (start 103.551 97.911037) (end 102.273807 96.633844) (width 0.3) (layer "F.Cu") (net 6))
 (segment (start 99.07 102.755) (end 99.675 102.755) (width 0.3) (layer "F.Cu") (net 6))
 (segment (start 100.925 97.254) (end 99.07 97.254) (width 0.3) (layer "F.Cu") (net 6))
 (segment (start 100.93 102.759) (end 101.530109 103.359109) (width 0.3) (layer "F.Cu") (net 6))
 (segment (start 103.551 102.169401) (end 103.551 97.911037) (width 0.3) (layer "F.Cu") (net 6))
 (segment (start 102.361292 103.359109) (end 103.551 102.169401) (width 0.3) (layer "F.Cu") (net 6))
 (segment (start 102.273807 96.633844) (end 100.933844 96.633844) (width 0.3) (layer "F.Cu") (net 6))
 (segment (start 99.68 102.76) (end 100.93 102.76) (width 0.3) (layer "F.Cu") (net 6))
 (segment (start 100.93 97.259) (end 100.925 97.254) (width 0.3) (layer "F.Cu") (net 6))
 (segment (start 95.01 106.34) (end 95 106.35) (width 0.3) (layer "F.Cu") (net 6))
 (segment (start 101.530109 103.359109) (end 102.361292 103.359109) (width 0.3) (layer "F.Cu") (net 6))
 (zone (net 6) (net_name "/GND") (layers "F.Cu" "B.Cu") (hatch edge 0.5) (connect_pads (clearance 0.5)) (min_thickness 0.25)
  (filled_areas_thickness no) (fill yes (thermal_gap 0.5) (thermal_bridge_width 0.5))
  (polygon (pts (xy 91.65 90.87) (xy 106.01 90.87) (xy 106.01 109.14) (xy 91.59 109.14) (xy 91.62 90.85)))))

